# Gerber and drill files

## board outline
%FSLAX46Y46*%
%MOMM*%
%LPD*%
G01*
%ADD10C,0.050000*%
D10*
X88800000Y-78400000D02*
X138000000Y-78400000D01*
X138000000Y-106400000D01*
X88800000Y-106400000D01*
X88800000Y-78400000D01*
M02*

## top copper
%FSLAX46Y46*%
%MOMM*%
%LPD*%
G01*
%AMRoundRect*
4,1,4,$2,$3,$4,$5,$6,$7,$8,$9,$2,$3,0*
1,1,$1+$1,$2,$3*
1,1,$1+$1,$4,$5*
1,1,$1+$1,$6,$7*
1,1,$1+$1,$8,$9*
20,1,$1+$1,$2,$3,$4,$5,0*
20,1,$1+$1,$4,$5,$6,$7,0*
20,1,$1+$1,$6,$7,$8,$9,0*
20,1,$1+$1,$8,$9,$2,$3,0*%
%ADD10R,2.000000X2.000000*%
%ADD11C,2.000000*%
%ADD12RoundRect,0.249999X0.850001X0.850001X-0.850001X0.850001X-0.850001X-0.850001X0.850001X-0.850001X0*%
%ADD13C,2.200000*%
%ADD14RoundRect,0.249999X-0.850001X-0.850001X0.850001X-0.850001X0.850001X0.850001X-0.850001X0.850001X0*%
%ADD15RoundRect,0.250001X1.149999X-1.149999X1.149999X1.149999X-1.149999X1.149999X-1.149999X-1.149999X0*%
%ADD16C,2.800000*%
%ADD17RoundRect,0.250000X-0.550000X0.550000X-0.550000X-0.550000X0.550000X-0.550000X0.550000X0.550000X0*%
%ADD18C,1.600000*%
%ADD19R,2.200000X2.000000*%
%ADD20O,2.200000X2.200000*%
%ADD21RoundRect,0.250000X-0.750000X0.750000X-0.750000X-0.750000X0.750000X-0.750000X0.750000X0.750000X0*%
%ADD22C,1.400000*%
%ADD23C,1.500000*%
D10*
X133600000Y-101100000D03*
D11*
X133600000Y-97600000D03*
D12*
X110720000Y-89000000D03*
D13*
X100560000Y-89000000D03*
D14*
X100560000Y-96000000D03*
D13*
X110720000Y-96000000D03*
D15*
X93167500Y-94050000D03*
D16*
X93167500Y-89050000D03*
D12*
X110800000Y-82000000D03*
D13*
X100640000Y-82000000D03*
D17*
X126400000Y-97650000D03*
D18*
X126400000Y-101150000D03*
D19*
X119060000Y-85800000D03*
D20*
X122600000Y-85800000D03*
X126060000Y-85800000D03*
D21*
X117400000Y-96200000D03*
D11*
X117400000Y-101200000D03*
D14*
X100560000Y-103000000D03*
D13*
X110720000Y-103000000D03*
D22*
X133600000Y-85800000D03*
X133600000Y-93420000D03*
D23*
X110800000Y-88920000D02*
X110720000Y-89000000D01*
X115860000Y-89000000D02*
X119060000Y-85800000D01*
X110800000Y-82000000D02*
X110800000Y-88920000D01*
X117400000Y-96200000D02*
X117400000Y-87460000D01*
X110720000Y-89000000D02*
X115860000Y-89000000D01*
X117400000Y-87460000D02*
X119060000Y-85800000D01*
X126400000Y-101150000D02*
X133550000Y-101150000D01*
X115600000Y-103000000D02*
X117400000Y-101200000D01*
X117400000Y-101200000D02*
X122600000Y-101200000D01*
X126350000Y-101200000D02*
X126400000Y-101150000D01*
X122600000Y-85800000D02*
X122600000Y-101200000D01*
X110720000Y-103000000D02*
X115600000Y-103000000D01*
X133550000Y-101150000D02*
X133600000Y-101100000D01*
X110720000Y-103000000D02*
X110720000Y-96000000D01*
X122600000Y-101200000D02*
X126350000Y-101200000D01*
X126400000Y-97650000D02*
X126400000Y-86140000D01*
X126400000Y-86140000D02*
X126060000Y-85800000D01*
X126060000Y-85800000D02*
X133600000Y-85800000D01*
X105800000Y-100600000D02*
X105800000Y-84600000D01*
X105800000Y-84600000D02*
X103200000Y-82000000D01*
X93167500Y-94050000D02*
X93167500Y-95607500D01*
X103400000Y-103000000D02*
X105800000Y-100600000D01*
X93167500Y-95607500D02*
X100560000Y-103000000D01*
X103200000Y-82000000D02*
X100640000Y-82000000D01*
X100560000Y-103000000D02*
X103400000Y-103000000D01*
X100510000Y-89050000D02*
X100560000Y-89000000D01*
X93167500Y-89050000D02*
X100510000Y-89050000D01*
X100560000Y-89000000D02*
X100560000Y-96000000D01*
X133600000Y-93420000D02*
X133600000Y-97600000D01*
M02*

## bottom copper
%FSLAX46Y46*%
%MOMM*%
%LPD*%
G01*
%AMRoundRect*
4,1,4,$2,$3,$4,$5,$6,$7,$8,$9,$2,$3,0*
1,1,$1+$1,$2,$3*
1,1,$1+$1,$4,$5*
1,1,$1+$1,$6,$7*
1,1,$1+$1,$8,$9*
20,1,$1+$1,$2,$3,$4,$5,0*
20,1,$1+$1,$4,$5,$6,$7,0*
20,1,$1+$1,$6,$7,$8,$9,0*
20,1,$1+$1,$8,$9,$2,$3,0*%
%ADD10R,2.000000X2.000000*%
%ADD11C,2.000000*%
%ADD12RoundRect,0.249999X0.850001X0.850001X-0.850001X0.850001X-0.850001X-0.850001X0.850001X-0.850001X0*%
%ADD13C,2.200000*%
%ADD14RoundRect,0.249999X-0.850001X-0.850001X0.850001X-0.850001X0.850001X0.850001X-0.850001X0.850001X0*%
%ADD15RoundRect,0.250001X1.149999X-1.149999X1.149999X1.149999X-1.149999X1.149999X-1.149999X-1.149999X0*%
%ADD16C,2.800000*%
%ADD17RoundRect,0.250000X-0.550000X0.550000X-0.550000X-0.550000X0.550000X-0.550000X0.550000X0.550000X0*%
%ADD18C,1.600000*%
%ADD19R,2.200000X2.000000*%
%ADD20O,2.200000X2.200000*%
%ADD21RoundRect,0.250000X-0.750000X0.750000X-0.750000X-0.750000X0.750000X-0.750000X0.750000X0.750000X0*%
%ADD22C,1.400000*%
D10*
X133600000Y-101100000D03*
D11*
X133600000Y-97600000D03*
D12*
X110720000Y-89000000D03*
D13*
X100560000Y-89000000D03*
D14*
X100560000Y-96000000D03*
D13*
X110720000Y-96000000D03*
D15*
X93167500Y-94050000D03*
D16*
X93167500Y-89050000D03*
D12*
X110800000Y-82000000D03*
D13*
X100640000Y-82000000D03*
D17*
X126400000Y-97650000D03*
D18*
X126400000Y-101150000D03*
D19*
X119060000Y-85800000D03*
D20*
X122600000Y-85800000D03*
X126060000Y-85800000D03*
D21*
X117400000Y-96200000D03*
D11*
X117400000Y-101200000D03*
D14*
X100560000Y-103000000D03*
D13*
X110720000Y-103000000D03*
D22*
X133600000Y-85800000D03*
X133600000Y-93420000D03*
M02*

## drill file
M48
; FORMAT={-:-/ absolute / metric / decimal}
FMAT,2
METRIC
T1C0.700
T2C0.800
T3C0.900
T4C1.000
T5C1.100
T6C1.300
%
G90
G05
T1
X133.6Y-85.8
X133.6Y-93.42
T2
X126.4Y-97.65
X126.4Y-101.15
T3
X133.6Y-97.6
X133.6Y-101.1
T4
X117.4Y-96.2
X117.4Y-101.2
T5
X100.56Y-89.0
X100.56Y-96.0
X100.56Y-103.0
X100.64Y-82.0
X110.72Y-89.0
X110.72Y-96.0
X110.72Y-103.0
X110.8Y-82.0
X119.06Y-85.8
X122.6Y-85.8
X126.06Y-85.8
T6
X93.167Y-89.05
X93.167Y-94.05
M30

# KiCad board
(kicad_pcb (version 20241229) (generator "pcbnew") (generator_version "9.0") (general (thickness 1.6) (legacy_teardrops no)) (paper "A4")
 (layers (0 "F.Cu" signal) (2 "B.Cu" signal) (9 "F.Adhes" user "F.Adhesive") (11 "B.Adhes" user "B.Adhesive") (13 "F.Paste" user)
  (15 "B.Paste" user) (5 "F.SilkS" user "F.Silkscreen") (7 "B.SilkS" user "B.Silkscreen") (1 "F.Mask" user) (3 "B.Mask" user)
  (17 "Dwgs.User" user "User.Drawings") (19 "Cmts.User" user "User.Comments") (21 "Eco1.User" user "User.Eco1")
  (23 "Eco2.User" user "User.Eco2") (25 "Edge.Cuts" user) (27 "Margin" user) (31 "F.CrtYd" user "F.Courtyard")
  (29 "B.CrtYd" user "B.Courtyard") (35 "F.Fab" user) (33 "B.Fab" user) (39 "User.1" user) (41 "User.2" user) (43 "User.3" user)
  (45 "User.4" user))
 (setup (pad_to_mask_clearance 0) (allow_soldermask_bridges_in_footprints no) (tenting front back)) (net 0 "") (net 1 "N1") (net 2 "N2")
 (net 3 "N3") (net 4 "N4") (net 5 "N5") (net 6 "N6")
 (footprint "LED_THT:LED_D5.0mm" (layer "F.Cu") (at 133.6 100.6 90)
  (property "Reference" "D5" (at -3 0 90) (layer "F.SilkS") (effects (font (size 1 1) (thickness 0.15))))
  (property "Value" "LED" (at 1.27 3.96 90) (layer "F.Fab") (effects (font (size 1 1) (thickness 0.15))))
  (pad "1" thru_hole rect (at -0.5 0 90) (size 2 2) (drill 0.9) (layers "*.Cu" "*.Mask") (remove_unused_layers no) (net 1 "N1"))
  (pad "2" thru_hole circle (at 3 0 90) (size 2 2) (drill 0.9) (layers "*.Cu" "*.Mask") (remove_unused_layers no) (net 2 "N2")))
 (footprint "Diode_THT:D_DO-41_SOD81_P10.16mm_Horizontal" (layer "F.Cu") (at 110.72 89 180)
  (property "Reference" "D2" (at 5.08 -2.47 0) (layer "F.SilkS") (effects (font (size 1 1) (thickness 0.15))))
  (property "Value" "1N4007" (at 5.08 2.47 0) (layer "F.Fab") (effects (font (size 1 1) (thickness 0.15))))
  (pad "1" thru_hole roundrect (at 0 0 180) (size 2.2 2.2) (drill 1.1) (layers "*.Cu" "*.Mask") (remove_unused_layers no)
   (roundrect_rratio 0.113636) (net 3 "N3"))
  (pad "2" thru_hole circle (at 10.16 0 180) (size 2.2 2.2) (drill 1.1) (layers "*.Cu" "*.Mask") (remove_unused_layers no) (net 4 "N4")))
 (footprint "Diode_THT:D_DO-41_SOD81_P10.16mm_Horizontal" (layer "F.Cu") (at 100.56 96)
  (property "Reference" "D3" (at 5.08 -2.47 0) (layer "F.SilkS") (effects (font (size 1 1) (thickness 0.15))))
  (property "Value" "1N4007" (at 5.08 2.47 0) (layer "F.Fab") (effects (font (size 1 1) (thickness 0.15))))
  (pad "1" thru_hole roundrect (at 0 0) (size 2.2 2.2) (drill 1.1) (layers "*.Cu" "*.Mask") (remove_unused_layers no)
   (roundrect_rratio 0.113636) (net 4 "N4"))
  (pad "2" thru_hole circle (at 10.16 0) (size 2.2 2.2) (drill 1.1) (layers "*.Cu" "*.Mask") (remove_unused_layers no) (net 1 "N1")))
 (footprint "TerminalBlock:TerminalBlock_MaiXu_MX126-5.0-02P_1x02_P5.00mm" (layer "F.Cu") (at 93.1675 94.05 90)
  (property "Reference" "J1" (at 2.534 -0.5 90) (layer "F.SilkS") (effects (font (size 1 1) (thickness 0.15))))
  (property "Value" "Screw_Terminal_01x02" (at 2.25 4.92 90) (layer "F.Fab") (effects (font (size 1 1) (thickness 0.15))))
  (pad "1" thru_hole roundrect (at 0 0 90) (size 2.8 2.8) (drill 1.3) (layers "*.Cu" "*.Mask") (remove_unused_layers no)
   (roundrect_rratio 0.089286) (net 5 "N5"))
  (pad "2" thru_hole circle (at 5 0 90) (size 2.8 2.8) (drill 1.3) (layers "*.Cu" "*.Mask") (remove_unused_layers no) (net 4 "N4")))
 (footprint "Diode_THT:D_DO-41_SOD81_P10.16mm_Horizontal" (layer "F.Cu") (at 110.8 82 180)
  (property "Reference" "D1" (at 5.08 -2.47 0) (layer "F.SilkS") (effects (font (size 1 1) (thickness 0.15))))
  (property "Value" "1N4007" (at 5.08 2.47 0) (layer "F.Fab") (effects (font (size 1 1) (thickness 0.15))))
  (pad "1" thru_hole roundrect (at 0 0 180) (size 2.2 2.2) (drill 1.1) (layers "*.Cu" "*.Mask") (remove_unused_layers no)
   (roundrect_rratio 0.113636) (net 3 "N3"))
  (pad "2" thru_hole circle (at 10.16 0 180) (size 2.2 2.2) (drill 1.1) (layers "*.Cu" "*.Mask") (remove_unused_layers no) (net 5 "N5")))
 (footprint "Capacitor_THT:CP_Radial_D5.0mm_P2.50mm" (layer "F.Cu") (at 126.4 98.15 -90)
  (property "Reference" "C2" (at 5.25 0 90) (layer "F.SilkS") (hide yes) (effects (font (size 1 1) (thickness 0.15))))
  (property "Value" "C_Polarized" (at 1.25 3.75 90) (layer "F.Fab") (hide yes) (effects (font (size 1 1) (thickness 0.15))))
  (pad "1" thru_hole roundrect (at -0.5 0 270) (size 1.6 1.6) (drill 0.8) (layers "*.Cu" "*.Mask") (remove_unused_layers no)
   (roundrect_rratio 0.15625) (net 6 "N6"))
  (pad "2" thru_hole circle (at 3 0 270) (size 1.6 1.6) (drill 0.8) (layers "*.Cu" "*.Mask") (remove_unused_layers no) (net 1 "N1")))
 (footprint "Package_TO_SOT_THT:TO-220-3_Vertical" (layer "F.Cu") (at 120.06 85.8)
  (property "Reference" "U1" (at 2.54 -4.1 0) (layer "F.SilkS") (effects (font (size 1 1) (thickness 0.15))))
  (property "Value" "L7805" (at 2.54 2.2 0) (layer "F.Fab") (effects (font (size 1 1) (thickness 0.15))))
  (pad "1" thru_hole rect (at -1 0) (size 2.2 2) (drill 1.1) (layers "*.Cu" "*.Mask") (remove_unused_layers no) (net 3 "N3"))
  (pad "2" thru_hole oval (at 2.54 0) (size 2.2 2.2) (drill 1.1) (layers "*.Cu" "*.Mask") (remove_unused_layers no) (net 1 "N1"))
  (pad "3" thru_hole oval (at 6 0) (size 2.2 2.2) (drill 1.1) (layers "*.Cu" "*.Mask") (remove_unused_layers no) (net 6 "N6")))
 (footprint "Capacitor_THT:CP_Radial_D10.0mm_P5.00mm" (layer "F.Cu") (at 117.4 96.2 -90)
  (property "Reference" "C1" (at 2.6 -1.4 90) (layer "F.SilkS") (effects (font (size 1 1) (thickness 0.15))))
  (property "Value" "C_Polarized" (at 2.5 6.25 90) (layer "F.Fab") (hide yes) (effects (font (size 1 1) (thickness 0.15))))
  (pad "1" thru_hole roundrect (at 0 0 270) (size 2 2) (drill 1) (layers "*.Cu" "*.Mask") (remove_unused_layers no) (roundrect_rratio 0.125)
   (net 3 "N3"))
  (pad "2" thru_hole circle (at 5 0 270) (size 2 2) (drill 1) (layers "*.Cu" "*.Mask") (remove_unused_layers no) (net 1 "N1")))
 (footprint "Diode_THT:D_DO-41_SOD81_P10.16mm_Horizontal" (layer "F.Cu") (at 100.56 103)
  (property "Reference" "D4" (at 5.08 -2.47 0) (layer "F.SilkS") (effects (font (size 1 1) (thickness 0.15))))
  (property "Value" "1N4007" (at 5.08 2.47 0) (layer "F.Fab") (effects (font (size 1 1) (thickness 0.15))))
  (pad "1" thru_hole roundrect (at 0 0) (size 2.2 2.2) (drill 1.1) (layers "*.Cu" "*.Mask") (remove_unused_layers no)
   (roundrect_rratio 0.113636) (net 5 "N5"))
  (pad "2" thru_hole circle (at 10.16 0) (size 2.2 2.2) (drill 1.1) (layers "*.Cu" "*.Mask") (remove_unused_layers no) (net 1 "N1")))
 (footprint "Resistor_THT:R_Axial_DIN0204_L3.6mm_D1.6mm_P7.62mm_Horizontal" (layer "F.Cu") (at 133.6 85.8 -90)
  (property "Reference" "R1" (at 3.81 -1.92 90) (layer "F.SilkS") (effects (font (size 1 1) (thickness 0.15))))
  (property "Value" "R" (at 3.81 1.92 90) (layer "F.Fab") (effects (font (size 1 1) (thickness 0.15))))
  (pad "1" thru_hole circle (at 0 0 270) (size 1.4 1.4) (drill 0.7) (layers "*.Cu" "*.Mask") (remove_unused_layers no) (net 6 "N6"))
  (pad "2" thru_hole circle (at 7.62 0 270) (size 1.4 1.4) (drill 0.7) (layers "*.Cu" "*.Mask") (remove_unused_layers no) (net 2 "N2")))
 (gr_rect (start 88.8 78.4) (end 138 106.4) (stroke (width 0.05) (type solid)) (fill no) (layer "Edge.Cuts"))
 (segment (start 110.8 88.92) (end 110.72 89) (width 1.5) (layer "F.Cu") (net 3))
 (segment (start 115.86 89) (end 119.06 85.8) (width 1.5) (layer "F.Cu") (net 3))
 (segment (start 110.8 82) (end 110.8 88.92) (width 1.5) (layer "F.Cu") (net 3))
 (segment (start 117.4 96.2) (end 117.4 87.46) (width 1.5) (layer "F.Cu") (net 3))
 (segment (start 110.72 89) (end 115.86 89) (width 1.5) (layer "F.Cu") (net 3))
 (segment (start 117.4 87.46) (end 119.06 85.8) (width 1.5) (layer "F.Cu") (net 3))
 (segment (start 126.4 101.15) (end 133.55 101.15) (width 1.5) (layer "F.Cu") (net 1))
 (segment (start 115.6 103) (end 117.4 101.2) (width 1.5) (layer "F.Cu") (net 1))
 (segment (start 117.4 101.2) (end 122.6 101.2) (width 1.5) (layer "F.Cu") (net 1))
 (segment (start 126.35 101.2) (end 126.4 101.15) (width 1.5) (layer "F.Cu") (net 1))
 (segment (start 122.6 85.8) (end 122.6 101.2) (width 1.5) (layer "F.Cu") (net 1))
 (segment (start 110.72 103) (end 115.6 103) (width 1.5) (layer "F.Cu") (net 1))
 (segment (start 133.55 101.15) (end 133.6 101.1) (width 1.5) (layer "F.Cu") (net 1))
 (segment (start 110.72 103) (end 110.72 96) (width 1.5) (layer "F.Cu") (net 1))
 (segment (start 122.6 101.2) (end 126.35 101.2) (width 1.5) (layer "F.Cu") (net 1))
 (segment (start 126.4 97.65) (end 126.4 86.14) (width 1.5) (layer "F.Cu") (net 6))
 (segment (start 126.4 86.14) (end 126.06 85.8) (width 1.5) (layer "F.Cu") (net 6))
 (segment (start 126.06 85.8) (end 133.6 85.8) (width 1.5) (layer "F.Cu") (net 6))
 (segment (start 105.8 100.6) (end 105.8 84.6) (width 1.5) (layer "F.Cu") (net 5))
 (segment (start 105.8 84.6) (end 103.2 82) (width 1.5) (layer "F.Cu") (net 5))
 (segment (start 93.1675 94.05) (end 93.1675 95.6075) (width 1.5) (layer "F.Cu") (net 5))
 (segment (start 103.4 103) (end 105.8 100.6) (width 1.5) (layer "F.Cu") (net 5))
 (segment (start 93.1675 95.6075) (end 100.56 103) (width 1.5) (layer "F.Cu") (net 5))
 (segment (start 103.2 82) (end 100.64 82) (width 1.5) (layer "F.Cu") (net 5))
 (segment (start 100.56 103) (end 103.4 103) (width 1.5) (layer "F.Cu") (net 5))
 (segment (start 100.51 89.05) (end 100.56 89) (width 1.5) (layer "F.Cu") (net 4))
 (segment (start 93.1675 89.05) (end 100.51 89.05) (width 1.5) (layer "F.Cu") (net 4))
 (segment (start 100.56 89) (end 100.56 96) (width 1.5) (layer "F.Cu") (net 4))
 (segment (start 133.6 93.42) (end 133.6 97.6) (width 1.5) (layer "F.Cu") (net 2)))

